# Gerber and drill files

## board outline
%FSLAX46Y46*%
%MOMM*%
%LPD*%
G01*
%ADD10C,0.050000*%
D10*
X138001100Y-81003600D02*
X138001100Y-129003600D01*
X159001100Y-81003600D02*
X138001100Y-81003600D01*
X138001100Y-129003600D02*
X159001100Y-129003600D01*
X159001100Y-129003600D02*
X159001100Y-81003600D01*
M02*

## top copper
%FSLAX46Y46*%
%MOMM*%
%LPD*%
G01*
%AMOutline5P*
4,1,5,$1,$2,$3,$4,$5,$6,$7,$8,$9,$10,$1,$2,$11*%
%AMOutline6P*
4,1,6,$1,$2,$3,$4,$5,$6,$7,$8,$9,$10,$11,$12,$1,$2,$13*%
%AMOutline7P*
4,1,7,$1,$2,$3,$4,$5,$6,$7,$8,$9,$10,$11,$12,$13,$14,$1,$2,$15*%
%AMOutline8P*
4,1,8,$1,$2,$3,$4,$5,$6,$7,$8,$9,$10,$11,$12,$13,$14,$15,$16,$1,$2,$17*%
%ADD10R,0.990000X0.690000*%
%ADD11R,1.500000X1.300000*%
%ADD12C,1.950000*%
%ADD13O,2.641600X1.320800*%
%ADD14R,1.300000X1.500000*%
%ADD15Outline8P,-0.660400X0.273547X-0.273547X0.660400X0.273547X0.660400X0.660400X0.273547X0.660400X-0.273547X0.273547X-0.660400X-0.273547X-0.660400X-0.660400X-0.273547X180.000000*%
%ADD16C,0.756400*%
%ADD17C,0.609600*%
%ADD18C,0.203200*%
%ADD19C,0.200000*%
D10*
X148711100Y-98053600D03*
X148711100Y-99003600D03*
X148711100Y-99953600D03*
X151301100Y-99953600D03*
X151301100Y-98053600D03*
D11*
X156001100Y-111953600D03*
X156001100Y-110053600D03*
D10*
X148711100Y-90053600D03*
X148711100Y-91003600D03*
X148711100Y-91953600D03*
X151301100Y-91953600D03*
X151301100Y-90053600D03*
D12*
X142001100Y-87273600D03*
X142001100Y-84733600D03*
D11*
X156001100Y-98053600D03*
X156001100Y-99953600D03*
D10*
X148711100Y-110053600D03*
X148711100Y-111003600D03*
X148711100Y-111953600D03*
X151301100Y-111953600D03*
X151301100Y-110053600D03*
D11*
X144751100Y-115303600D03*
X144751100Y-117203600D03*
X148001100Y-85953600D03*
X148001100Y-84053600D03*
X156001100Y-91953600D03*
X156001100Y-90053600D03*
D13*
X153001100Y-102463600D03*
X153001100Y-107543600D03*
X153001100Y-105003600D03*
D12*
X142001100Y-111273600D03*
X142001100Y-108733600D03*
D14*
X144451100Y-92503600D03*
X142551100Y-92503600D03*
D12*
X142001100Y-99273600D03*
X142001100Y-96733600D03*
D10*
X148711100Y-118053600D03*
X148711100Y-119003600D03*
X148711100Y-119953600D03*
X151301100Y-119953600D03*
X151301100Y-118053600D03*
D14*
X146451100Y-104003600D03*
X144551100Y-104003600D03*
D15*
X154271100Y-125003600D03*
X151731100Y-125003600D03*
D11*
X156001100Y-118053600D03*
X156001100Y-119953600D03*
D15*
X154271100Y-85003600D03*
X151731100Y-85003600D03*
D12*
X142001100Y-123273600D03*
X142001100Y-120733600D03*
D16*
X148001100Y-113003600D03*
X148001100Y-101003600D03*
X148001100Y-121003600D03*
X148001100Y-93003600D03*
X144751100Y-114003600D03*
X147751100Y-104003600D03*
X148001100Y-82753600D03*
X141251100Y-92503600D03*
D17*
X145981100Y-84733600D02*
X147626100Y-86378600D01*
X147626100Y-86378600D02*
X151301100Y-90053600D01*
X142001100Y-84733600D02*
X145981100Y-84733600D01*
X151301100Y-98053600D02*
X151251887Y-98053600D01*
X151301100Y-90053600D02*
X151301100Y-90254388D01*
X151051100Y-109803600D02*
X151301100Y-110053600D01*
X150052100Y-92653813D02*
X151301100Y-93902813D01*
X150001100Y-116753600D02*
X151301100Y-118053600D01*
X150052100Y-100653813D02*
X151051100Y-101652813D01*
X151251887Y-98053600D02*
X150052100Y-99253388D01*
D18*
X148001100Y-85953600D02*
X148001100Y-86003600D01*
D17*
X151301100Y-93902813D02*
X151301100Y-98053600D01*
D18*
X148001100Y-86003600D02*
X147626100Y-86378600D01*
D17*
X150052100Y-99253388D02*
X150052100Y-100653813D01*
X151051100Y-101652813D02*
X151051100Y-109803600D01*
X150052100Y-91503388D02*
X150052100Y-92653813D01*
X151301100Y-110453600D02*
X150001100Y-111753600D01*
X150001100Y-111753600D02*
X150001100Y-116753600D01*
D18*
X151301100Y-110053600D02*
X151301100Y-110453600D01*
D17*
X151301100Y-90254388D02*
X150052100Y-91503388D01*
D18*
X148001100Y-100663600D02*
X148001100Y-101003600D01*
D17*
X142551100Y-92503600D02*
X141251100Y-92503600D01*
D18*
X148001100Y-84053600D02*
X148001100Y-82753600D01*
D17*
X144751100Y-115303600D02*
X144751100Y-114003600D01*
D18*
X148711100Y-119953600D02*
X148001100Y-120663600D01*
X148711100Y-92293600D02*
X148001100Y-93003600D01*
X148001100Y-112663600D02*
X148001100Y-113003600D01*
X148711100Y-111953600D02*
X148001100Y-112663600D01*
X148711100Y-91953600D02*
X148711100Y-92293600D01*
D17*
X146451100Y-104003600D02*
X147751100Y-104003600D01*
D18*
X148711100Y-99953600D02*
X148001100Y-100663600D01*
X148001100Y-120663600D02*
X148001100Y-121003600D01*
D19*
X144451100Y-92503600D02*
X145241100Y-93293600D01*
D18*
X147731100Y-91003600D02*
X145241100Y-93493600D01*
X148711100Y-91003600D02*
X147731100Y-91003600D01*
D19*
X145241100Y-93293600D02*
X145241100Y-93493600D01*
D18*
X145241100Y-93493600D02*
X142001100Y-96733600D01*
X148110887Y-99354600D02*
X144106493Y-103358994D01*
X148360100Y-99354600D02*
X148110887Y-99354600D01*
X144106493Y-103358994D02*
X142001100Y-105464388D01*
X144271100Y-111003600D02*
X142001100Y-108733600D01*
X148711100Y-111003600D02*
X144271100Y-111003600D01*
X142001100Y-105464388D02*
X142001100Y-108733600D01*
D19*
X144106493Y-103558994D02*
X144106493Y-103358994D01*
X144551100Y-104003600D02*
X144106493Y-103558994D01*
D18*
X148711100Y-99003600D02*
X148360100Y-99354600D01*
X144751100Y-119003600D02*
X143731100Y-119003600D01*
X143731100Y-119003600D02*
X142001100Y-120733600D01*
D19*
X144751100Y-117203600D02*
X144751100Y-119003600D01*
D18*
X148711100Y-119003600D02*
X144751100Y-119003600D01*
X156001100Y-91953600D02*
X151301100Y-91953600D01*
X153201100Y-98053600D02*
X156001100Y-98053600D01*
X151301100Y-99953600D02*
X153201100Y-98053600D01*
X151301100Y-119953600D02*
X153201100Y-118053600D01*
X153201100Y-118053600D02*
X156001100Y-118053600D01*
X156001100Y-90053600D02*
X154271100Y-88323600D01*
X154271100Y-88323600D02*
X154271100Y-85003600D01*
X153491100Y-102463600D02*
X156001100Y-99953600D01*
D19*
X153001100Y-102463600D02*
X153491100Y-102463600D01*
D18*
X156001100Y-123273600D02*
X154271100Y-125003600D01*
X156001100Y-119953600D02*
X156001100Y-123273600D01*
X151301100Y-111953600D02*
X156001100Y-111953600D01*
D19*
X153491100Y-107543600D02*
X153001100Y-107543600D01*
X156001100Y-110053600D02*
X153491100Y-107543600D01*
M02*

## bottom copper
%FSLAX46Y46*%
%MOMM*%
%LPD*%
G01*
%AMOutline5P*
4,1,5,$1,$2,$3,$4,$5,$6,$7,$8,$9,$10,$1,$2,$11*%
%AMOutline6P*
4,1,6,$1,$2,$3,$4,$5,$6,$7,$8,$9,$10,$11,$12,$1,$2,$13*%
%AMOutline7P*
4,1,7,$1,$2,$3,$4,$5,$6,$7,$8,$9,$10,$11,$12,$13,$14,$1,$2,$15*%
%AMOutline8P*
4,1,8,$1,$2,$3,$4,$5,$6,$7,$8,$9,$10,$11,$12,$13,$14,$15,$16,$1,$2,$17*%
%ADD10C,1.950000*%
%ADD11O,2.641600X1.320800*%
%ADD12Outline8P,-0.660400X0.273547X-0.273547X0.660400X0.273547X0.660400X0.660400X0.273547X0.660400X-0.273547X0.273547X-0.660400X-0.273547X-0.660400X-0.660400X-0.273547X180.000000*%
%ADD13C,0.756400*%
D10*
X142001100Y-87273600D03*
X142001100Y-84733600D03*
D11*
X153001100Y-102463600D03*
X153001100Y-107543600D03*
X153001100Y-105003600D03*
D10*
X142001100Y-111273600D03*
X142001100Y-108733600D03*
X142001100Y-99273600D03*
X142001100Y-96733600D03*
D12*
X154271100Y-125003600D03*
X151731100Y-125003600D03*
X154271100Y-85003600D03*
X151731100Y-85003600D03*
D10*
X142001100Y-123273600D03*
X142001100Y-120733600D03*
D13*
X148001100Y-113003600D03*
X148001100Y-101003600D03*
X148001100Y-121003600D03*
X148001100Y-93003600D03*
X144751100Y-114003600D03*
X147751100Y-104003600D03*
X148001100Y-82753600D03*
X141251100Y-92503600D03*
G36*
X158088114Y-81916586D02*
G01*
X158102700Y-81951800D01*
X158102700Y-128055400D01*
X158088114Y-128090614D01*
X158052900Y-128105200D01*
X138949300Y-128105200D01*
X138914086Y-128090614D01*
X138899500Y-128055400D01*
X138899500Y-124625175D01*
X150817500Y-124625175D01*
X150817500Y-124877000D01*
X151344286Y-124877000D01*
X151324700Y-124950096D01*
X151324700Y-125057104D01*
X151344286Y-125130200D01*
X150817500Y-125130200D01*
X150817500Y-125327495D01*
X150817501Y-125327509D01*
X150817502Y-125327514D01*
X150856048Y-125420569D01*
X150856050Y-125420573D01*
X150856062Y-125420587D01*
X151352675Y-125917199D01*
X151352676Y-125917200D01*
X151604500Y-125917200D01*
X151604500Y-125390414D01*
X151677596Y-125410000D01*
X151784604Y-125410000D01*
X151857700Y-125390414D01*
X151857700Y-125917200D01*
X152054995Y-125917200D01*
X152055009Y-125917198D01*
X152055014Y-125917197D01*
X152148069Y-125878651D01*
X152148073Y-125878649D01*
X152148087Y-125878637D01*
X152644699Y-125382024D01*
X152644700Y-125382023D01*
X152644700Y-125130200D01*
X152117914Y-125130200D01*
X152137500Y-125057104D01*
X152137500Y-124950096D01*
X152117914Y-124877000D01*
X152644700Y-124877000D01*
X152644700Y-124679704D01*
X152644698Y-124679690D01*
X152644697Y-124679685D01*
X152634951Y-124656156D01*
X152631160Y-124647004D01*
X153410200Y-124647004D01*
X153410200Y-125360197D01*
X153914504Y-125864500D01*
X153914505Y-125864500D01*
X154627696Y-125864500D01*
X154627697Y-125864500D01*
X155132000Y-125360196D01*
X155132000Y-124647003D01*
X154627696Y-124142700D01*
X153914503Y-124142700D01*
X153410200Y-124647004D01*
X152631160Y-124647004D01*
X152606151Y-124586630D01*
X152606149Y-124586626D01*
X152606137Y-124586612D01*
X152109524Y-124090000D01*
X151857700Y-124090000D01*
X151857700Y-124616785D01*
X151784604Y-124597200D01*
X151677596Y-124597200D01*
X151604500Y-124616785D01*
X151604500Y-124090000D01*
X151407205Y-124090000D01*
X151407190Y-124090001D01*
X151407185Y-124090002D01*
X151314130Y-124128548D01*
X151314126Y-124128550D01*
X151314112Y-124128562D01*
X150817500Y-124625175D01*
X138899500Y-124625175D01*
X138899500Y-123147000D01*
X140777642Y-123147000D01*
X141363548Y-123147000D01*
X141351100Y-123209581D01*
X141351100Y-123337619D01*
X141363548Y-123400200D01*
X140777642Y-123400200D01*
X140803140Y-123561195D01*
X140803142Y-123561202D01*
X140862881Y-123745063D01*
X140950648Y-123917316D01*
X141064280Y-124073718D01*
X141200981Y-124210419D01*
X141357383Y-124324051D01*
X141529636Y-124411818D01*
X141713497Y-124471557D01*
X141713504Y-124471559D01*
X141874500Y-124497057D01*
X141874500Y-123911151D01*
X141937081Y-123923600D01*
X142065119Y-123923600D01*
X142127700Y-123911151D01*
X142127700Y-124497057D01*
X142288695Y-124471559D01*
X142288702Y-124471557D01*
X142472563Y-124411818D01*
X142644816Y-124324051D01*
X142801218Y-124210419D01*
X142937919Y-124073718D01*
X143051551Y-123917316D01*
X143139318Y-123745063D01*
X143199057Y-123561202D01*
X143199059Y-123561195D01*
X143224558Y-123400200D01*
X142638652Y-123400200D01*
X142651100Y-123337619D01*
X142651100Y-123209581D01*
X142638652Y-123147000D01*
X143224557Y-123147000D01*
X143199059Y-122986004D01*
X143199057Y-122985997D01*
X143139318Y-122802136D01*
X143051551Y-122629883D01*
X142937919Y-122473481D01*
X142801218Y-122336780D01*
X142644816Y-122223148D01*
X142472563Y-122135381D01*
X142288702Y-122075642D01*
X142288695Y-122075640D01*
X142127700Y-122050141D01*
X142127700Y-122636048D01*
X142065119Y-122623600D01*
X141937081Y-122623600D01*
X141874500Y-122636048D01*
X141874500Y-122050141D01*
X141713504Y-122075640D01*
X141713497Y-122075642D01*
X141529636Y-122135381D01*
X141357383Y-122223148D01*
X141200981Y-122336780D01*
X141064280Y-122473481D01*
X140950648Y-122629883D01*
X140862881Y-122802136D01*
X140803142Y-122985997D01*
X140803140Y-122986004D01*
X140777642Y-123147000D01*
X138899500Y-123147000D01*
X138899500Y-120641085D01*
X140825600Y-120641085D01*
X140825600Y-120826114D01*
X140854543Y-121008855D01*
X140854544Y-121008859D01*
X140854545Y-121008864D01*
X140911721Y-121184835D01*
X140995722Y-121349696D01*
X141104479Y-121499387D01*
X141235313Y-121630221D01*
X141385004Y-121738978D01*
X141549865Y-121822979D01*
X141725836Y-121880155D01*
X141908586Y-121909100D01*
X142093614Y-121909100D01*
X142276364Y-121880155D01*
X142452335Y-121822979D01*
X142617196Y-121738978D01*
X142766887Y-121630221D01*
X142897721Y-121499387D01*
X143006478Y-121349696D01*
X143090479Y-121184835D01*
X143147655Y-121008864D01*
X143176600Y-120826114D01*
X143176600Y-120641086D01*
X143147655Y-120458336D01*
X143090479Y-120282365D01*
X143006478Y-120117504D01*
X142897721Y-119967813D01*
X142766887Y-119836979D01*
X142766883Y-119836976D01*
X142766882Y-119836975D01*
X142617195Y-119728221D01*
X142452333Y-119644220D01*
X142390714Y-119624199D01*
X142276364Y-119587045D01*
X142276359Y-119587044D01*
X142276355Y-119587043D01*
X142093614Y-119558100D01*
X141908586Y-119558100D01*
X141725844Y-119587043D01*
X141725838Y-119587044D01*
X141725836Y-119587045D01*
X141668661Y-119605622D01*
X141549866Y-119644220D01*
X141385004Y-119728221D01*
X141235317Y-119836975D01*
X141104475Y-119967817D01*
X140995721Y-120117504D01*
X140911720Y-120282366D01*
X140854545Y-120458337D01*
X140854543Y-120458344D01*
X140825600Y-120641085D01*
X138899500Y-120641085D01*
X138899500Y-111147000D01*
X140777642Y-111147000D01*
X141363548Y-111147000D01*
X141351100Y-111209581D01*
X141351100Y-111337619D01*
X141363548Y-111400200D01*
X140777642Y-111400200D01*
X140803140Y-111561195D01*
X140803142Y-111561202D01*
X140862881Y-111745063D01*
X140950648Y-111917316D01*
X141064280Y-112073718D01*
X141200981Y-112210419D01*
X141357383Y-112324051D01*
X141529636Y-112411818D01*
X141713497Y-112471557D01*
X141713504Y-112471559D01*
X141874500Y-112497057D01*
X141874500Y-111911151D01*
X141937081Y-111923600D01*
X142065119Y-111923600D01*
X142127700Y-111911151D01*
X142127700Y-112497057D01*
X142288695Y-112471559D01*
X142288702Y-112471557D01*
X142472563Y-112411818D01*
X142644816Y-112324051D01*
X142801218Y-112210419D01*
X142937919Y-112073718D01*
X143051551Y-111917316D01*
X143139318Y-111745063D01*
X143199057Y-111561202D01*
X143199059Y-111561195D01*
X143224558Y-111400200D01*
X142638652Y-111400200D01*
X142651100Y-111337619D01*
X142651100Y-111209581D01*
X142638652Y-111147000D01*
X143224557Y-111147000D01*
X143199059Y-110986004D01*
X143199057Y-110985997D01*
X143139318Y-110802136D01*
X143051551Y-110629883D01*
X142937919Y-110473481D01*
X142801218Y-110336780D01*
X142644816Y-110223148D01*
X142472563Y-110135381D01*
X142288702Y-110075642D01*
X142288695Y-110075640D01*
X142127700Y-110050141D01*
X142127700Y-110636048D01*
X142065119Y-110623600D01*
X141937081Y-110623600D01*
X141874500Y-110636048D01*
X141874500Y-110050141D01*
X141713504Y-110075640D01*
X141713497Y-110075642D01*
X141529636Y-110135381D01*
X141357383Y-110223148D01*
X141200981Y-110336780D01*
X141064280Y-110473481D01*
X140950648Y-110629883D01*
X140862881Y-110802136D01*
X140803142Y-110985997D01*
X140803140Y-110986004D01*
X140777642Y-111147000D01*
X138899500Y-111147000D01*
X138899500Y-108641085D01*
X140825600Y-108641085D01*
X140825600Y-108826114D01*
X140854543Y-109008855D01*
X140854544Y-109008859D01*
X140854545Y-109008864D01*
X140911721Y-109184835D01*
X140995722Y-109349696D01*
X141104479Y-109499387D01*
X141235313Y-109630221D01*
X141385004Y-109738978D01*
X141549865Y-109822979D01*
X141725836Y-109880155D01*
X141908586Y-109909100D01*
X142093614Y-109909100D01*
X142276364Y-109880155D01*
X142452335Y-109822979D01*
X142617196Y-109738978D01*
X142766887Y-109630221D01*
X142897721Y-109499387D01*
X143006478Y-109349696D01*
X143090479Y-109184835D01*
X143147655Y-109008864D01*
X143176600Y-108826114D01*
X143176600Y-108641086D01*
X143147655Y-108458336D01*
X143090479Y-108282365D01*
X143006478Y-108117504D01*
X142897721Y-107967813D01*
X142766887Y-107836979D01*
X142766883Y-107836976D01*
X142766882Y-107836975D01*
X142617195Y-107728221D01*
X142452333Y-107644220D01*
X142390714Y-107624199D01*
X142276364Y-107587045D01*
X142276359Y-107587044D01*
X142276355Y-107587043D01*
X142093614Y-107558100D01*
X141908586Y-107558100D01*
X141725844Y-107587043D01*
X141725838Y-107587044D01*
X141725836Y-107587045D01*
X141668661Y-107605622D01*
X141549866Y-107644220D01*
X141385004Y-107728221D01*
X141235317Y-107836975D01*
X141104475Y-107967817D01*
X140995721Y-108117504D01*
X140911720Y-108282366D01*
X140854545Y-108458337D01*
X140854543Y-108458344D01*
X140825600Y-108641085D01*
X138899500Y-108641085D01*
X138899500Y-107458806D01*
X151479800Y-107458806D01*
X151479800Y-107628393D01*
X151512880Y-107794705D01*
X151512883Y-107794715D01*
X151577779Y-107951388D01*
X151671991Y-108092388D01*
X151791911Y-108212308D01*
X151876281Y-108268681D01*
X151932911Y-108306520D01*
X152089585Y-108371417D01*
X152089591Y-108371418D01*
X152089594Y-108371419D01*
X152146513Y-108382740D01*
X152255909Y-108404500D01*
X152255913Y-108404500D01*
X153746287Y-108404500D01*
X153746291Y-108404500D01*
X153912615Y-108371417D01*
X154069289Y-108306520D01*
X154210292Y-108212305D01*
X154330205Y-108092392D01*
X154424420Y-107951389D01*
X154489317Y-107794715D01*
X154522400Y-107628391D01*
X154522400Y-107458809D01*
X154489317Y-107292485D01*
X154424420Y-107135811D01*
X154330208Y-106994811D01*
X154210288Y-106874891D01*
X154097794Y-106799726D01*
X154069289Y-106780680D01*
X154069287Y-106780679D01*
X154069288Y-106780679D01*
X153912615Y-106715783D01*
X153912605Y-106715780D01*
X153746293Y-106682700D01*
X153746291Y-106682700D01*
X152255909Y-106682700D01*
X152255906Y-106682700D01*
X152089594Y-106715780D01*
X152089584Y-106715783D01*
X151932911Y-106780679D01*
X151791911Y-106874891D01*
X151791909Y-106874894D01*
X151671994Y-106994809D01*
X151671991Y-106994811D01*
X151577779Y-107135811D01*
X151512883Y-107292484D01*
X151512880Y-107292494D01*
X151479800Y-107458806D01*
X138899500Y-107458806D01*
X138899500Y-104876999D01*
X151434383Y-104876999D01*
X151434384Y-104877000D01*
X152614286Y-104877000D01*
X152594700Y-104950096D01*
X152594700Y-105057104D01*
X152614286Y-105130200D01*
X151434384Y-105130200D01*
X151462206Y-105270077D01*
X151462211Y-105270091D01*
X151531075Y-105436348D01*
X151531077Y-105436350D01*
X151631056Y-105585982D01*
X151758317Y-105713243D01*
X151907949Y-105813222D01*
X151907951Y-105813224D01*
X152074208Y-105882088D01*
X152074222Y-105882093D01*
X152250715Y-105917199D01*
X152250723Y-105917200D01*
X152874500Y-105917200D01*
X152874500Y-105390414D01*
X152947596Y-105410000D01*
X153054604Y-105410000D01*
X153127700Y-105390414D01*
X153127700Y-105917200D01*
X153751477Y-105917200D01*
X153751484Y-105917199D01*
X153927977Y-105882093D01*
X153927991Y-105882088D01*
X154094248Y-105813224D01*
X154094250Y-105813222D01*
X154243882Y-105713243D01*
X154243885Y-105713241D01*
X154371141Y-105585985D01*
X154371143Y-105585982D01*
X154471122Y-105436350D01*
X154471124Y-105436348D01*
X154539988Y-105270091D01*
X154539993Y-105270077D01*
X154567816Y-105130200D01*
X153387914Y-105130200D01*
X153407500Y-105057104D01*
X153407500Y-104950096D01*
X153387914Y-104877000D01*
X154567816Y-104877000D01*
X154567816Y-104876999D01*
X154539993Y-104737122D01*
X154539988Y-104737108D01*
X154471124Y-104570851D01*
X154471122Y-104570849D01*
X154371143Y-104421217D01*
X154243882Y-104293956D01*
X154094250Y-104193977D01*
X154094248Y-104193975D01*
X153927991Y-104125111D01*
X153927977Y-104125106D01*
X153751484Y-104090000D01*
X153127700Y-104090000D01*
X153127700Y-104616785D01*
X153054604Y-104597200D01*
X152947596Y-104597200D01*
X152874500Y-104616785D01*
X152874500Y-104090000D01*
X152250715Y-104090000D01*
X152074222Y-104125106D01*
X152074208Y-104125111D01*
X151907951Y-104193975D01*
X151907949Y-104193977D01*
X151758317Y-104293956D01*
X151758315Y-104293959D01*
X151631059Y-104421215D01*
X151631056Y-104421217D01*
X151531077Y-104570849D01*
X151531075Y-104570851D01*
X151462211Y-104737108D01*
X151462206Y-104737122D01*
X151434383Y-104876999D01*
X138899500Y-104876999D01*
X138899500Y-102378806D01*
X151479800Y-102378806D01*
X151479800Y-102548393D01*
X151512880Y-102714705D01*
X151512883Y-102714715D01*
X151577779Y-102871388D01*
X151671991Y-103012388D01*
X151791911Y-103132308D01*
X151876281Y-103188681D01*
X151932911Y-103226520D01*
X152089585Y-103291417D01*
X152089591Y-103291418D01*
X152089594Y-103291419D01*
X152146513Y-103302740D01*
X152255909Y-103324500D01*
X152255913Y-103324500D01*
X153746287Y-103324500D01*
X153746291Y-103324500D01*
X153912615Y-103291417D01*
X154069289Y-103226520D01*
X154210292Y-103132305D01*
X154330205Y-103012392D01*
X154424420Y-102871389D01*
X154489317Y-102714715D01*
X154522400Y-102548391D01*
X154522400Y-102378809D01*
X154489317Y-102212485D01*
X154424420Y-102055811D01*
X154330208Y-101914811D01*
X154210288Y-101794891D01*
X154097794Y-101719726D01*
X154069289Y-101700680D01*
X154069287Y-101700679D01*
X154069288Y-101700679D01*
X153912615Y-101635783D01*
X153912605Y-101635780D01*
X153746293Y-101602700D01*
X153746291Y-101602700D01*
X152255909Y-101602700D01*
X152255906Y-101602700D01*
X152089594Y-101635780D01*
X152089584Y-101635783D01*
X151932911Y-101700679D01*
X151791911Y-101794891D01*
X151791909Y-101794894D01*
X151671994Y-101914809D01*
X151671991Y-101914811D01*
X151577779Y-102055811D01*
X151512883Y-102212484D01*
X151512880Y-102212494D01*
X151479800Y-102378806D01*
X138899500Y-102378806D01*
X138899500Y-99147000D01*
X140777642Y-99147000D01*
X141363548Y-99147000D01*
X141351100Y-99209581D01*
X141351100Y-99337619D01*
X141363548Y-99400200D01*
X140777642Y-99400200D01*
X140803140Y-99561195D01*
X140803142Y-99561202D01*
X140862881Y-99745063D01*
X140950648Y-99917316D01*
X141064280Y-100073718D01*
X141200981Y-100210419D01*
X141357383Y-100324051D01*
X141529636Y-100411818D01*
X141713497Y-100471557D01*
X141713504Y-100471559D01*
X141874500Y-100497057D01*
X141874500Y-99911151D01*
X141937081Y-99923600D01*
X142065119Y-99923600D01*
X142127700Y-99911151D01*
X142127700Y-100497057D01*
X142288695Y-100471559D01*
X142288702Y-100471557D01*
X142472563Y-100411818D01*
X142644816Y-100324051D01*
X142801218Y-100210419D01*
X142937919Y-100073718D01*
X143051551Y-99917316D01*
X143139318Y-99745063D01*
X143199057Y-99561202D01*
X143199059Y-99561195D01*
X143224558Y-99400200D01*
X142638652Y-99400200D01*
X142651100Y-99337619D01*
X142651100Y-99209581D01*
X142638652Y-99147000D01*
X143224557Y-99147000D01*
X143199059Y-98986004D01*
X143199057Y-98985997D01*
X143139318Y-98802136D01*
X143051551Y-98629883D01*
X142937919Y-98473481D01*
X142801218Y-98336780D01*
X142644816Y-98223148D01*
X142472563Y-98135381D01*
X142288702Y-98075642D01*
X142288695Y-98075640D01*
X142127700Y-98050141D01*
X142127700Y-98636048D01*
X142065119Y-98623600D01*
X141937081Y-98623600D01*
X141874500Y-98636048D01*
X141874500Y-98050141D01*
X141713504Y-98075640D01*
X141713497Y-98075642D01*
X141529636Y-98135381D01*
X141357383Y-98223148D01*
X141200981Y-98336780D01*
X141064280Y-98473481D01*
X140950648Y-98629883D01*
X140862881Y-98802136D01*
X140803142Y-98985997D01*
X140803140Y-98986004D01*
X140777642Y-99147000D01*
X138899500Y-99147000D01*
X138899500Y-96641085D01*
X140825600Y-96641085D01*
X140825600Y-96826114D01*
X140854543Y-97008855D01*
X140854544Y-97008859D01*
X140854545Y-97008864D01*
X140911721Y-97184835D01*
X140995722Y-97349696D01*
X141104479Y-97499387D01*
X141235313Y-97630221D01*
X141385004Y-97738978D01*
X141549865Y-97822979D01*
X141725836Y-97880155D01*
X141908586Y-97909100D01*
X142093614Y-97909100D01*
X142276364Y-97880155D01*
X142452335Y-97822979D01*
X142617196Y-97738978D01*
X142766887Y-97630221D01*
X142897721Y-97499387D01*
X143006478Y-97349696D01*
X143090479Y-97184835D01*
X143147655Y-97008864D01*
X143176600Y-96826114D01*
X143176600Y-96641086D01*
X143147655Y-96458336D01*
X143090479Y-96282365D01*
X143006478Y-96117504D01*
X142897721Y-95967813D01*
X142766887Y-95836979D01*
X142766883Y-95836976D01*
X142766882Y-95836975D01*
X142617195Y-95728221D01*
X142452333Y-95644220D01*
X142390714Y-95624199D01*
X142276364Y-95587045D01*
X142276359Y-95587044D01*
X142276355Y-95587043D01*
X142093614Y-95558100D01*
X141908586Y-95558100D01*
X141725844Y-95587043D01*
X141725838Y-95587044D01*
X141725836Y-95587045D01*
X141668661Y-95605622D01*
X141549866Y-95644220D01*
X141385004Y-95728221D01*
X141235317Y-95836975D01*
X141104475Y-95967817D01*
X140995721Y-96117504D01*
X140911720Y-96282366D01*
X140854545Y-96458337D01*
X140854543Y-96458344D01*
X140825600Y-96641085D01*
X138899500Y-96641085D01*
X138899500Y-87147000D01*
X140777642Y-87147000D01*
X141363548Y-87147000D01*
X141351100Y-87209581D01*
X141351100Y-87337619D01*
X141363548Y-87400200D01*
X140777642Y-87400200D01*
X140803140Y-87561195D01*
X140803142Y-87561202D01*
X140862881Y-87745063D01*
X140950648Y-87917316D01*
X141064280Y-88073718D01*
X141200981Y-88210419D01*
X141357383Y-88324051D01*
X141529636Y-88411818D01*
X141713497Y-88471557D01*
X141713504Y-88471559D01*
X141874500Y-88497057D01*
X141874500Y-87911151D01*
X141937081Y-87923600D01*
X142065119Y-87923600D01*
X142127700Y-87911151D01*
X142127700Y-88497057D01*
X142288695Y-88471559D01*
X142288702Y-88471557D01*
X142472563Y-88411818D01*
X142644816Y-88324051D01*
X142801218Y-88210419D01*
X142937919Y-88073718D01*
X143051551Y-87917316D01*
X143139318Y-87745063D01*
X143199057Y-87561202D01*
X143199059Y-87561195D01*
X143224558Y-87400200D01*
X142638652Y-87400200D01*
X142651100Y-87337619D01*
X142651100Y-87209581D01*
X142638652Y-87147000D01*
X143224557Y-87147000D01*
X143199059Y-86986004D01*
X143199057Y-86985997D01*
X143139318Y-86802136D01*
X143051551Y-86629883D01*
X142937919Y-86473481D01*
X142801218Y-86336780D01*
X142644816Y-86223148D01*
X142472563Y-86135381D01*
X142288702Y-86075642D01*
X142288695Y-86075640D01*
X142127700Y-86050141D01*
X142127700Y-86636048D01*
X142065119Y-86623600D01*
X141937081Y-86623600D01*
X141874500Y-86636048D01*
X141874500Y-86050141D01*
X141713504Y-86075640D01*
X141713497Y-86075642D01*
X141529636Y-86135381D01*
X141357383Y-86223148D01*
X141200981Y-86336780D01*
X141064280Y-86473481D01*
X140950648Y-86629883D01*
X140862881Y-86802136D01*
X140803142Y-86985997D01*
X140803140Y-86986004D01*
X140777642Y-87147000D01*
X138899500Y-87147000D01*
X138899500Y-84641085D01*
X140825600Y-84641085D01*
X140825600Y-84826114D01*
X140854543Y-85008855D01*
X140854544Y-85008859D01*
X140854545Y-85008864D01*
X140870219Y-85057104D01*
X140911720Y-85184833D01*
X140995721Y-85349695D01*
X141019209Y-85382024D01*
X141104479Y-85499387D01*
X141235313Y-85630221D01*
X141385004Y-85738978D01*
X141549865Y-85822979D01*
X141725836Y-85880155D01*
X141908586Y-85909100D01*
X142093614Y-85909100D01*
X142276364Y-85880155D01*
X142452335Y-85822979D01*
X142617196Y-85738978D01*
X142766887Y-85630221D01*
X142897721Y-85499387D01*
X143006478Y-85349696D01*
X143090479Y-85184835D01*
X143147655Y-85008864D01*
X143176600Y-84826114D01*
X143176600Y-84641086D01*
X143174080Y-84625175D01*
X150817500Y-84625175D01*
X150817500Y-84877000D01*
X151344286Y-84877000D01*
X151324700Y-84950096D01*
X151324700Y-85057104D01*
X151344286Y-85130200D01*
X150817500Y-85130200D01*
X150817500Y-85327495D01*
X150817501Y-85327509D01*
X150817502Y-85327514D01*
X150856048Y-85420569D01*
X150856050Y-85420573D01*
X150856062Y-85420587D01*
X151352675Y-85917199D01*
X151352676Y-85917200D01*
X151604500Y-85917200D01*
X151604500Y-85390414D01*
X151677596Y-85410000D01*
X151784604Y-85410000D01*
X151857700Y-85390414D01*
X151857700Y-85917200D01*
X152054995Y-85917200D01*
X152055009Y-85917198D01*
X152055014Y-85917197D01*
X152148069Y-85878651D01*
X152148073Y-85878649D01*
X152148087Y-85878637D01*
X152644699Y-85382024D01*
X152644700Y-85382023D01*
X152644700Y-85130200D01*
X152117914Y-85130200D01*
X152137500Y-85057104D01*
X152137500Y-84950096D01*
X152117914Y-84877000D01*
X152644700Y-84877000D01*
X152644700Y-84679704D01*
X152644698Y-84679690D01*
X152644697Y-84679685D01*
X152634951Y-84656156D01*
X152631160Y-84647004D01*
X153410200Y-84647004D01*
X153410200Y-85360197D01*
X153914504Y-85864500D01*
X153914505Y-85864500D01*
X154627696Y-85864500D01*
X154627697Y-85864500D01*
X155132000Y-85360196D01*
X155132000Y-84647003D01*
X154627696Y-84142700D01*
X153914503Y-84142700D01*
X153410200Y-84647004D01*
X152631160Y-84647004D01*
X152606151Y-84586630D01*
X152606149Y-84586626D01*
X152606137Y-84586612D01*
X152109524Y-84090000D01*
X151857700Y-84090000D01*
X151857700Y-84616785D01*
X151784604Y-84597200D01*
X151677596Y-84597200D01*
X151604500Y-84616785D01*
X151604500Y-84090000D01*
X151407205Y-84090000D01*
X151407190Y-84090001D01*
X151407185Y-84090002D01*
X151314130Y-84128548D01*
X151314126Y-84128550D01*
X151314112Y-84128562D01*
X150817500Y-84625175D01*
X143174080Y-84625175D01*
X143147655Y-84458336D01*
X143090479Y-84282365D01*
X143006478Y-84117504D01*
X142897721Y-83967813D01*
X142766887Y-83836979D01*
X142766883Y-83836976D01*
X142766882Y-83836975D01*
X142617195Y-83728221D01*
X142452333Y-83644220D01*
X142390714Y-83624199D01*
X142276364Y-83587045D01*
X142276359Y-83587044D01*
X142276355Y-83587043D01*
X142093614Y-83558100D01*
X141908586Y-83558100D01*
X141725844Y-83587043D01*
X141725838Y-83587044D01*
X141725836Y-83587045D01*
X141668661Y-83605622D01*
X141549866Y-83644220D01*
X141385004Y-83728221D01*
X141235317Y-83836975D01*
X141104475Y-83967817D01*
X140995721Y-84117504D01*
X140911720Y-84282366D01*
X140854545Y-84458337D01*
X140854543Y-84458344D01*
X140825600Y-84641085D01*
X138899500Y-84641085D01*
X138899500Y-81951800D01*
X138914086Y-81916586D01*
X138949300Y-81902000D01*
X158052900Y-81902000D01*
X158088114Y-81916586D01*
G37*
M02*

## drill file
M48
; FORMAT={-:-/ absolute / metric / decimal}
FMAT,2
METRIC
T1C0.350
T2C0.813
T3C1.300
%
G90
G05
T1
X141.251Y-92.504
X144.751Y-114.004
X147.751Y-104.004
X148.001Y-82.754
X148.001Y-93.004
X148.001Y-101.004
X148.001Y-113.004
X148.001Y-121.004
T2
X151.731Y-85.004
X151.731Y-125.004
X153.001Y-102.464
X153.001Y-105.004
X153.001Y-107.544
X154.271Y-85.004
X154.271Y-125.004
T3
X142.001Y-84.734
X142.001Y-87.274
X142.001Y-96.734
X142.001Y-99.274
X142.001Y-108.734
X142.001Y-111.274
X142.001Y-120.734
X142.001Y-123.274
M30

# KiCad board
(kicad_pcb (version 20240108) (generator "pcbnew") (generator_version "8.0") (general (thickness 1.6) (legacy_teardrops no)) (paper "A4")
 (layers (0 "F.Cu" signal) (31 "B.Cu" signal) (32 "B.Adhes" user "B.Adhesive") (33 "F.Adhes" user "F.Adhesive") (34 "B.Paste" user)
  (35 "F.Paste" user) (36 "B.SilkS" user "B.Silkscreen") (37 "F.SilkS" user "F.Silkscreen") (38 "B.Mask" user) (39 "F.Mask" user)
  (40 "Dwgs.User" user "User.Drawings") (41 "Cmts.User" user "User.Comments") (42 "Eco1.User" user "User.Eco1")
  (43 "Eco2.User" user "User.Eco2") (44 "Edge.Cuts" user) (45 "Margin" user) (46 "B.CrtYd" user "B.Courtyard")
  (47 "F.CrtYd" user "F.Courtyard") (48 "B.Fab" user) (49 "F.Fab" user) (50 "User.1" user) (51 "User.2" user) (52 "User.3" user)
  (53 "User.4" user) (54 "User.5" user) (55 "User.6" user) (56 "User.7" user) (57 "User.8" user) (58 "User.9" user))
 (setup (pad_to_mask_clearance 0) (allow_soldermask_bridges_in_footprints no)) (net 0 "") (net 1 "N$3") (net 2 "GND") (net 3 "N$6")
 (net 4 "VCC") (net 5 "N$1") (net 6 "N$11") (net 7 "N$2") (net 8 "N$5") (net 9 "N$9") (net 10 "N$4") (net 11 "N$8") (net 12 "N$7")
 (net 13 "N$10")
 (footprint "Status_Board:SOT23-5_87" (layer "F.Cu") (at 150.0011 99.0036 -90)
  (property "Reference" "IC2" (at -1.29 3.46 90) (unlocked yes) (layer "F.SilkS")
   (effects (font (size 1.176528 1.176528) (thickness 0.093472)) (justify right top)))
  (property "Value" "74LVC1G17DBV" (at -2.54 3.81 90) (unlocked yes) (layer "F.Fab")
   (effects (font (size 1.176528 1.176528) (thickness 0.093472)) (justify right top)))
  (pad "1" smd rect (at -0.95 1.29 270) (size 0.69 0.99) (layers "F.Cu" "F.Paste" "F.Mask") (solder_mask_margin 0.1016)
   (thermal_bridge_angle 0))
  (pad "2" smd rect (at 0 1.29 270) (size 0.69 0.99) (layers "F.Cu" "F.Paste" "F.Mask") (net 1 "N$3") (solder_mask_margin 0.1016)
   (thermal_bridge_angle 0))
  (pad "3" smd rect (at 0.95 1.29 270) (size 0.69 0.99) (layers "F.Cu" "F.Paste" "F.Mask") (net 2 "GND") (solder_mask_margin 0.1016)
   (thermal_bridge_angle 0))
  (pad "4" smd rect (at 0.95 -1.3 270) (size 0.69 0.99) (layers "F.Cu" "F.Paste" "F.Mask") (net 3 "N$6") (solder_mask_margin 0.1016)
   (thermal_bridge_angle 0))
  (pad "5" smd rect (at -0.95 -1.3 270) (size 0.69 0.99) (layers "F.Cu" "F.Paste" "F.Mask") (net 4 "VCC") (solder_mask_margin 0.1016)
   (thermal_bridge_angle 0)))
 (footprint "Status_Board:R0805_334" (layer "F.Cu") (at 156.0011 111.0036 90)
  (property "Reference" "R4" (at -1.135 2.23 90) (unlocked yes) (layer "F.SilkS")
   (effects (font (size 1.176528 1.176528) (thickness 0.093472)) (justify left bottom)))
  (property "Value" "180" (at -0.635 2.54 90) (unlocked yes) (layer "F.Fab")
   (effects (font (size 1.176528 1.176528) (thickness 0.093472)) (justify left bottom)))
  (pad "1" smd rect (at -0.95 0 90) (size 1.3 1.5) (layers "F.Cu" "F.Paste" "F.Mask") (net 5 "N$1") (solder_mask_margin 0.1016)
   (thermal_bridge_angle 0))
  (pad "2" smd rect (at 0.95 0 90) (size 1.3 1.5) (layers "F.Cu" "F.Paste" "F.Mask") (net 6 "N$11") (solder_mask_margin 0.1016)
   (thermal_bridge_angle 0)))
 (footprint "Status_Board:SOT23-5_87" (layer "F.Cu") (at 150.0011 91.0036 -90)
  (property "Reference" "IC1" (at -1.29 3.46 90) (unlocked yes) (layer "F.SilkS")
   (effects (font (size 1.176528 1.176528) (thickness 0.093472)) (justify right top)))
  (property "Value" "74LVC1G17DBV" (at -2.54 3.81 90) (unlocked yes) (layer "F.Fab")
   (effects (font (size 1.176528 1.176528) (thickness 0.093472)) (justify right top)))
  (pad "1" smd rect (at -0.95 1.29 270) (size 0.69 0.99) (layers "F.Cu" "F.Paste" "F.Mask") (solder_mask_margin 0.1016)
   (thermal_bridge_angle 0))
  (pad "2" smd rect (at 0 1.29 270) (size 0.69 0.99) (layers "F.Cu" "F.Paste" "F.Mask") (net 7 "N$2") (solder_mask_margin 0.1016)
   (thermal_bridge_angle 0))
  (pad "3" smd rect (at 0.95 1.29 270) (size 0.69 0.99) (layers "F.Cu" "F.Paste" "F.Mask") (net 2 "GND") (solder_mask_margin 0.1016)
   (thermal_bridge_angle 0))
  (pad "4" smd rect (at 0.95 -1.3 270) (size 0.69 0.99) (layers "F.Cu" "F.Paste" "F.Mask") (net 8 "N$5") (solder_mask_margin 0.1016)
   (thermal_bridge_angle 0))
  (pad "5" smd rect (at -0.95 -1.3 270) (size 0.69 0.99) (layers "F.Cu" "F.Paste" "F.Mask") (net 4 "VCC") (solder_mask_margin 0.1016)
   (thermal_bridge_angle 0)))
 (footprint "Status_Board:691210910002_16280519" (layer "F.Cu") (at 142.0011 86.0036 90)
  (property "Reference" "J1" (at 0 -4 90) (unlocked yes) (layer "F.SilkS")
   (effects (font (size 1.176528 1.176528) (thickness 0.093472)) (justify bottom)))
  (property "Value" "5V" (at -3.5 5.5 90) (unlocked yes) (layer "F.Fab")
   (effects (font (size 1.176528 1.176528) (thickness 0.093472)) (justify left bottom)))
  (pad "1" thru_hole circle (at -1.27 0 90) (size 1.95 1.95) (drill 1.3) (layers "*.Cu" "*.Mask") (remove_unused_layers no) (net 2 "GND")
   (solder_mask_margin 0.1016) (thermal_bridge_angle 0))
  (pad "2" thru_hole circle (at 1.27 0 90) (size 1.95 1.95) (drill 1.3) (layers "*.Cu" "*.Mask") (remove_unused_layers no) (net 4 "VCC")
   (solder_mask_margin 0.1016) (thermal_bridge_angle 0)))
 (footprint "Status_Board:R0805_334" (layer "F.Cu") (at 156.0011 99.0036 -90)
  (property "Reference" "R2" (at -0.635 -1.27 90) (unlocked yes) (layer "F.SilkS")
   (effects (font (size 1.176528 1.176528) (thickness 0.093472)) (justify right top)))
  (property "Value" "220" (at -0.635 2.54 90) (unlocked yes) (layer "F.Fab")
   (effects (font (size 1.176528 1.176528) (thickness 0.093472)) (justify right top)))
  (pad "1" smd rect (at -0.95 0 270) (size 1.3 1.5) (layers "F.Cu" "F.Paste" "F.Mask") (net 3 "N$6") (solder_mask_margin 0.1016)
   (thermal_bridge_angle 0))
  (pad "2" smd rect (at 0.95 0 270) (size 1.3 1.5) (layers "F.Cu" "F.Paste" "F.Mask") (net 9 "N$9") (solder_mask_margin 0.1016)
   (thermal_bridge_angle 0)))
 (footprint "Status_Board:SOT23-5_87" (layer "F.Cu") (at 150.0011 111.0036 -90)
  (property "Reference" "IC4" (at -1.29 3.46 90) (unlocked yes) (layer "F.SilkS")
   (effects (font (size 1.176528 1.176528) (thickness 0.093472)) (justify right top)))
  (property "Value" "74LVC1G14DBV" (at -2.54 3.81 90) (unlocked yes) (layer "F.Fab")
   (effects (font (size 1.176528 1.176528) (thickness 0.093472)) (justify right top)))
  (pad "1" smd rect (at -0.95 1.29 270) (size 0.69 0.99) (layers "F.Cu" "F.Paste" "F.Mask") (solder_mask_margin 0.1016)
   (thermal_bridge_angle 0))
  (pad "2" smd rect (at 0 1.29 270) (size 0.69 0.99) (layers "F.Cu" "F.Paste" "F.Mask") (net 1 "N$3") (solder_mask_margin 0.1016)
   (thermal_bridge_angle 0))
  (pad "3" smd rect (at 0.95 1.29 270) (size 0.69 0.99) (layers "F.Cu" "F.Paste" "F.Mask") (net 2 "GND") (solder_mask_margin 0.1016)
   (thermal_bridge_angle 0))
  (pad "4" smd rect (at 0.95 -1.3 270) (size 0.69 0.99) (layers "F.Cu" "F.Paste" "F.Mask") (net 5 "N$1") (solder_mask_margin 0.1016)
   (thermal_bridge_angle 0))
  (pad "5" smd rect (at -0.95 -1.3 270) (size 0.69 0.99) (layers "F.Cu" "F.Paste" "F.Mask") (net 4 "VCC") (solder_mask_margin 0.1016)
   (thermal_bridge_angle 0)))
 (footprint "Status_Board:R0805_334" (layer "F.Cu") (at 144.7511 116.2536 -90)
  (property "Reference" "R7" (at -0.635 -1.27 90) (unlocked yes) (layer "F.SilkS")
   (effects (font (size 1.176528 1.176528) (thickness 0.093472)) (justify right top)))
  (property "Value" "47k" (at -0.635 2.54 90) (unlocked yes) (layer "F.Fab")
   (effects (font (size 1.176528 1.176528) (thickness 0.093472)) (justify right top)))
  (pad "1" smd rect (at -0.95 0 270) (size 1.3 1.5) (layers "F.Cu" "F.Paste" "F.Mask") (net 2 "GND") (solder_mask_margin 0.1016)
   (thermal_bridge_angle 0))
  (pad "2" smd rect (at 0.95 0 270) (size 1.3 1.5) (layers "F.Cu" "F.Paste" "F.Mask") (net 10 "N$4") (solder_mask_margin 0.1016)
   (thermal_bridge_angle 0)))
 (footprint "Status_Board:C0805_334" (layer "F.Cu") (at 148.0011 85.0036 90)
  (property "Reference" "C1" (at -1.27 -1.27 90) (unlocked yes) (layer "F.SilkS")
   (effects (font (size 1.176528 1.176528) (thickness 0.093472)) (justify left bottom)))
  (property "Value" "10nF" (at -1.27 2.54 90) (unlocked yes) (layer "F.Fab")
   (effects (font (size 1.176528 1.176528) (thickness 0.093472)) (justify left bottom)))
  (pad "1" smd rect (at -0.95 0 90) (size 1.3 1.5) (layers "F.Cu" "F.Paste" "F.Mask") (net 4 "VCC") (solder_mask_margin 0.1016)
   (thermal_bridge_angle 0))
  (pad "2" smd rect (at 0.95 0 90) (size 1.3 1.5) (layers "F.Cu" "F.Paste" "F.Mask") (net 2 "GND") (solder_mask_margin 0.1016)
   (thermal_bridge_angle 0)))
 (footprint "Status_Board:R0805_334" (layer "F.Cu") (at 156.0011 91.0036 90)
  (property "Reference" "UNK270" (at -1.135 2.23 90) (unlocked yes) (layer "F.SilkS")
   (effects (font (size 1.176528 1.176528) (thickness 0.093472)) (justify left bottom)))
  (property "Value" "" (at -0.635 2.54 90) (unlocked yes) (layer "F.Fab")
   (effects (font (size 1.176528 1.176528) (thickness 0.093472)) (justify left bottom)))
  (pad "1" smd rect (at -0.95 0 90) (size 1.3 1.5) (layers "F.Cu" "F.Paste" "F.Mask") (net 8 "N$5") (solder_mask_margin 0.1016)
   (thermal_bridge_angle 0))
  (pad "2" smd rect (at 0.95 0 90) (size 1.3 1.5) (layers "F.Cu" "F.Paste" "F.Mask") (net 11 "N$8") (solder_mask_margin 0.1016)
   (thermal_bridge_angle 0)))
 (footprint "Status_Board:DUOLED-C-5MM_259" (layer "F.Cu") (at 153.0011 105.0036 90)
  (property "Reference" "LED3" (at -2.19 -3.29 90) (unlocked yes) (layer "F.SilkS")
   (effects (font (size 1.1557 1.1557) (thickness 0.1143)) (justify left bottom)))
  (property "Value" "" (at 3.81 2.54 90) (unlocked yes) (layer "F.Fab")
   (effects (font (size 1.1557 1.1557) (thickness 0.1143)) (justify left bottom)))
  (pad "AR" thru_hole oval (at 2.54 0 180) (size 2.6416 1.3208) (drill 0.8128) (layers "*.Cu" "*.Mask") (remove_unused_layers no)
   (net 9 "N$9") (solder_mask_margin 0.1016) (thermal_bridge_angle 0))
  (pad "AX" thru_hole oval (at -2.54 0 180) (size 2.6416 1.3208) (drill 0.8128) (layers "*.Cu" "*.Mask") (remove_unused_layers no)
   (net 6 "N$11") (solder_mask_margin 0.1016) (thermal_bridge_angle 0))
  (pad "C" thru_hole oval (at 0 0 180) (size 2.6416 1.3208) (drill 0.8128) (layers "*.Cu" "*.Mask") (remove_unused_layers no) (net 2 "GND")
   (solder_mask_margin 0.1016) (thermal_bridge_angle 0)))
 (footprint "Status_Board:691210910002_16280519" (layer "F.Cu") (at 142.0011 110.0036 90)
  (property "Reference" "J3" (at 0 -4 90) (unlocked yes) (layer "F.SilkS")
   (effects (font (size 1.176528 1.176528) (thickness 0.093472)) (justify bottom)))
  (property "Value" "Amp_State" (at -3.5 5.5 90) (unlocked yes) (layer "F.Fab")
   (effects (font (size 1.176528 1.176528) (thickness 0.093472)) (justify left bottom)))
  (pad "1" thru_hole circle (at -1.27 0 90) (size 1.95 1.95) (drill 1.3) (layers "*.Cu" "*.Mask") (remove_unused_layers no) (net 2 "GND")
   (solder_mask_margin 0.1016) (thermal_bridge_angle 0))
  (pad "2" thru_hole circle (at 1.27 0 90) (size 1.95 1.95) (drill 1.3) (layers "*.Cu" "*.Mask") (remove_unused_layers no) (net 1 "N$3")
   (solder_mask_margin 0.1016) (thermal_bridge_angle 0)))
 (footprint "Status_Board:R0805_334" (layer "F.Cu") (at 143.5011 92.5036 180)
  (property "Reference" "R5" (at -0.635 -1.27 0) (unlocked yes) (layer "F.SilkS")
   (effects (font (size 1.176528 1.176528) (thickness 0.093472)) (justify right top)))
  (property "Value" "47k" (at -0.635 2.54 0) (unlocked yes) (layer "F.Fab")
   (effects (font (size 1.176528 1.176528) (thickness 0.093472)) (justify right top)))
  (pad "1" smd rect (at -0.95 0 180) (size 1.3 1.5) (layers "F.Cu" "F.Paste" "F.Mask") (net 7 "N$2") (solder_mask_margin 0.1016)
   (thermal_bridge_angle 0))
  (pad "2" smd rect (at 0.95 0 180) (size 1.3 1.5) (layers "F.Cu" "F.Paste" "F.Mask") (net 2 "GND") (solder_mask_margin 0.1016)
   (thermal_bridge_angle 0)))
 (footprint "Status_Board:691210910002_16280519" (layer "F.Cu") (at 142.0011 98.0036 90)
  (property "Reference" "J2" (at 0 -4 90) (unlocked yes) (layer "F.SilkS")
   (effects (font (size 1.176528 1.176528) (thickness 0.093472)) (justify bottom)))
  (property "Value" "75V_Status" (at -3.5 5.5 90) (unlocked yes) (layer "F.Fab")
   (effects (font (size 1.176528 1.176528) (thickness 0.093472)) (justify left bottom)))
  (pad "1" thru_hole circle (at -1.27 0 90) (size 1.95 1.95) (drill 1.3) (layers "*.Cu" "*.Mask") (remove_unused_layers no) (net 2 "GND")
   (solder_mask_margin 0.1016) (thermal_bridge_angle 0))
  (pad "2" thru_hole circle (at 1.27 0 90) (size 1.95 1.95) (drill 1.3) (layers "*.Cu" "*.Mask") (remove_unused_layers no) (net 7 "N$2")
   (solder_mask_margin 0.1016) (thermal_bridge_angle 0)))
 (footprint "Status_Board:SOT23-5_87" (layer "F.Cu") (at 150.0011 119.0036 -90)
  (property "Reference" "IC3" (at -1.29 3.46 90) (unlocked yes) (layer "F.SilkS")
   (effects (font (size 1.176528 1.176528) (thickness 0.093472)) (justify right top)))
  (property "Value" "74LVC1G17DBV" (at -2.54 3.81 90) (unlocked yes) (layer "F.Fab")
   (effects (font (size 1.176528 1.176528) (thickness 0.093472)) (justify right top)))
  (pad "1" smd rect (at -0.95 1.29 270) (size 0.69 0.99) (layers "F.Cu" "F.Paste" "F.Mask") (solder_mask_margin 0.1016)
   (thermal_bridge_angle 0))
  (pad "2" smd rect (at 0 1.29 270) (size 0.69 0.99) (layers "F.Cu" "F.Paste" "F.Mask") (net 10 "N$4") (solder_mask_margin 0.1016)
   (thermal_bridge_angle 0))
  (pad "3" smd rect (at 0.95 1.29 270) (size 0.69 0.99) (layers "F.Cu" "F.Paste" "F.Mask") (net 2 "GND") (solder_mask_margin 0.1016)
   (thermal_bridge_angle 0))
  (pad "4" smd rect (at 0.95 -1.3 270) (size 0.69 0.99) (layers "F.Cu" "F.Paste" "F.Mask") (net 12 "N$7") (solder_mask_margin 0.1016)
   (thermal_bridge_angle 0))
  (pad "5" smd rect (at -0.95 -1.3 270) (size 0.69 0.99) (layers "F.Cu" "F.Paste" "F.Mask") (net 4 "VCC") (solder_mask_margin 0.1016)
   (thermal_bridge_angle 0)))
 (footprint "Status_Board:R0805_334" (layer "F.Cu") (at 145.5011 104.0036 180)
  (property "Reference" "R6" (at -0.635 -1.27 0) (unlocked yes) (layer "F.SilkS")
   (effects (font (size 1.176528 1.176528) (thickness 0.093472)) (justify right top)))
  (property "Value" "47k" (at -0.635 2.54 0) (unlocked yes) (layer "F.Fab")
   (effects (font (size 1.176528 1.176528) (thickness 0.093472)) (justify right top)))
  (pad "1" smd rect (at -0.95 0 180) (size 1.3 1.5) (layers "F.Cu" "F.Paste" "F.Mask") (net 2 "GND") (solder_mask_margin 0.1016)
   (thermal_bridge_angle 0))
  (pad "2" smd rect (at 0.95 0 180) (size 1.3 1.5) (layers "F.Cu" "F.Paste" "F.Mask") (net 1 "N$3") (solder_mask_margin 0.1016)
   (thermal_bridge_angle 0)))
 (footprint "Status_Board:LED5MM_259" (layer "F.Cu") (at 153.0011 125.0036 180)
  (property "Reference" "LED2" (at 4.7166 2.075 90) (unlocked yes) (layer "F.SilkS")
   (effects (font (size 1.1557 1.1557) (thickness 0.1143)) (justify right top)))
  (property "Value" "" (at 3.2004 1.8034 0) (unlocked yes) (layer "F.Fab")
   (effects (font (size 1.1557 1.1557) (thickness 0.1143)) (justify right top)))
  (pad "A" thru_hole roundrect (at -1.27 0 180) (size 1.3208 1.3208) (drill 0.8128) (layers "*.Cu" "*.Mask") (remove_unused_layers no)
   (roundrect_rratio 0.25) (chamfer_ratio 0.2928932188) (chamfer top_left top_right bottom_left bottom_right) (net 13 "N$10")
   (solder_mask_margin 0.1016) (thermal_bridge_angle 0))
  (pad "K" thru_hole roundrect (at 1.27 0 180) (size 1.3208 1.3208) (drill 0.8128) (layers "*.Cu" "*.Mask") (remove_unused_layers no)
   (roundrect_rratio 0.25) (chamfer_ratio 0.2928932188) (chamfer top_left top_right bottom_left bottom_right) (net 2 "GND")
   (solder_mask_margin 0.1016) (thermal_bridge_angle 0)))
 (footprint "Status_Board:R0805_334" (layer "F.Cu") (at 156.0011 119.0036 -90)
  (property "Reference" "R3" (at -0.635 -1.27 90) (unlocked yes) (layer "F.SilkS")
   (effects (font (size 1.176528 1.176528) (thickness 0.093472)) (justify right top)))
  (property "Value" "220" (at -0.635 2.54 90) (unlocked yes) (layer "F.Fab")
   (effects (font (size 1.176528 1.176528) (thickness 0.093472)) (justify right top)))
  (pad "1" smd rect (at -0.95 0 270) (size 1.3 1.5) (layers "F.Cu" "F.Paste" "F.Mask") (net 12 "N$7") (solder_mask_margin 0.1016)
   (thermal_bridge_angle 0))
  (pad "2" smd rect (at 0.95 0 270) (size 1.3 1.5) (layers "F.Cu" "F.Paste" "F.Mask") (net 13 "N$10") (solder_mask_margin 0.1016)
   (thermal_bridge_angle 0)))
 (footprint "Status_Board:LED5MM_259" (layer "F.Cu") (at 153.0011 85.0036 180)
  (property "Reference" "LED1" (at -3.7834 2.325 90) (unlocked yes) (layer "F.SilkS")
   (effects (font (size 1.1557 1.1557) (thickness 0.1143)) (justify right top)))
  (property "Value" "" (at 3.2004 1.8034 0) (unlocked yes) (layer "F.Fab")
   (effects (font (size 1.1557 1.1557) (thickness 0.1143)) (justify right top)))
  (pad "A" thru_hole roundrect (at -1.27 0 180) (size 1.3208 1.3208) (drill 0.8128) (layers "*.Cu" "*.Mask") (remove_unused_layers no)
   (roundrect_rratio 0.25) (chamfer_ratio 0.2928932188) (chamfer top_left top_right bottom_left bottom_right) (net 11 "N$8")
   (solder_mask_margin 0.1016) (thermal_bridge_angle 0))
  (pad "K" thru_hole roundrect (at 1.27 0 180) (size 1.3208 1.3208) (drill 0.8128) (layers "*.Cu" "*.Mask") (remove_unused_layers no)
   (roundrect_rratio 0.25) (chamfer_ratio 0.2928932188) (chamfer top_left top_right bottom_left bottom_right) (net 2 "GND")
   (solder_mask_margin 0.1016) (thermal_bridge_angle 0)))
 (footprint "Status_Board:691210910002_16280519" (layer "F.Cu") (at 142.0011 122.0036 90)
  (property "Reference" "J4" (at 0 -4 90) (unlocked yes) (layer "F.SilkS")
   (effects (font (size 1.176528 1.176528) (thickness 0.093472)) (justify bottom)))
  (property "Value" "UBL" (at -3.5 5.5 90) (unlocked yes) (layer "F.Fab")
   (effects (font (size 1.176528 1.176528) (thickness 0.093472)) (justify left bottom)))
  (pad "1" thru_hole circle (at -1.27 0 90) (size 1.95 1.95) (drill 1.3) (layers "*.Cu" "*.Mask") (remove_unused_layers no) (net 2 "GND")
   (solder_mask_margin 0.1016) (thermal_bridge_angle 0))
  (pad "2" thru_hole circle (at 1.27 0 90) (size 1.95 1.95) (drill 1.3) (layers "*.Cu" "*.Mask") (remove_unused_layers no) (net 10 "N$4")
   (solder_mask_margin 0.1016) (thermal_bridge_angle 0)))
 (gr_line (start 138.0011 81.0036) (end 138.0011 129.0036) (stroke (width 0.05) (type solid)) (layer "Edge.Cuts"))
 (gr_line (start 159.0011 81.0036) (end 138.0011 81.0036) (stroke (width 0.05) (type solid)) (layer "Edge.Cuts"))
 (gr_line (start 138.0011 129.0036) (end 159.0011 129.0036) (stroke (width 0.05) (type solid)) (layer "Edge.Cuts"))
 (gr_line (start 159.0011 129.0036) (end 159.0011 81.0036) (stroke (width 0.05) (type solid)) (layer "Edge.Cuts"))
 (segment (start 145.9811 84.7336) (end 147.6261 86.3786) (width 0.6096) (layer "F.Cu") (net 4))
 (segment (start 147.6261 86.3786) (end 151.3011 90.0536) (width 0.6096) (layer "F.Cu") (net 4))
 (segment (start 142.0011 84.7336) (end 145.9811 84.7336) (width 0.6096) (layer "F.Cu") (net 4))
 (segment (start 151.3011 98.0536) (end 151.251887 98.0536) (width 0.6096) (layer "F.Cu") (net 4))
 (segment (start 151.3011 90.0536) (end 151.3011 90.254388) (width 0.6096) (layer "F.Cu") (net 4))
 (segment (start 151.0511 109.8036) (end 151.3011 110.0536) (width 0.6096) (layer "F.Cu") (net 4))
 (segment (start 150.0521 92.653813) (end 151.3011 93.902813) (width 0.6096) (layer "F.Cu") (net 4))
 (segment (start 150.0011 116.7536) (end 151.3011 118.0536) (width 0.6096) (layer "F.Cu") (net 4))
 (segment (start 150.0521 100.653813) (end 151.0511 101.652813) (width 0.6096) (layer "F.Cu") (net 4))
 (segment (start 151.251887 98.0536) (end 150.0521 99.253388) (width 0.6096) (layer "F.Cu") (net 4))
 (segment (start 148.0011 85.9536) (end 148.0011 86.0036) (width 0.2032) (layer "F.Cu") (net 4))
 (segment (start 151.3011 93.902813) (end 151.3011 98.0536) (width 0.6096) (layer "F.Cu") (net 4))
 (segment (start 148.0011 86.0036) (end 147.6261 86.3786) (width 0.2032) (layer "F.Cu") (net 4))
 (segment (start 150.0521 99.253388) (end 150.0521 100.653813) (width 0.6096) (layer "F.Cu") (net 4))
 (segment (start 151.0511 101.652813) (end 151.0511 109.8036) (width 0.6096) (layer "F.Cu") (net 4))
 (segment (start 150.0521 91.503388) (end 150.0521 92.653813) (width 0.6096) (layer "F.Cu") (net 4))
 (segment (start 151.3011 110.4536) (end 150.0011 111.7536) (width 0.6096) (layer "F.Cu") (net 4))
 (segment (start 150.0011 111.7536) (end 150.0011 116.7536) (width 0.6096) (layer "F.Cu") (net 4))
 (segment (start 151.3011 110.0536) (end 151.3011 110.4536) (width 0.2032) (layer "F.Cu") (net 4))
 (segment (start 151.3011 90.254388) (end 150.0521 91.503388) (width 0.6096) (layer "F.Cu") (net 4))
 (segment (start 148.0011 100.6636) (end 148.0011 101.0036) (width 0.2032) (layer "F.Cu") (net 2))
 (segment (start 142.5511 92.5036) (end 141.2511 92.5036) (width 0.6096) (layer "F.Cu") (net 2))
 (segment (start 148.0011 84.0536) (end 148.0011 82.7536) (width 0.2032) (layer "F.Cu") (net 2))
 (segment (start 144.7511 115.3036) (end 144.7511 114.0036) (width 0.6096) (layer "F.Cu") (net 2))
 (segment (start 148.7111 119.9536) (end 148.0011 120.6636) (width 0.2032) (layer "F.Cu") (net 2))
 (segment (start 148.7111 92.2936) (end 148.0011 93.0036) (width 0.2032) (layer "F.Cu") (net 2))
 (segment (start 148.0011 112.6636) (end 148.0011 113.0036) (width 0.2032) (layer "F.Cu") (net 2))
 (segment (start 148.7111 111.9536) (end 148.0011 112.6636) (width 0.2032) (layer "F.Cu") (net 2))
 (segment (start 148.7111 91.9536) (end 148.7111 92.2936) (width 0.2032) (layer "F.Cu") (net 2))
 (segment (start 146.4511 104.0036) (end 147.7511 104.0036) (width 0.6096) (layer "F.Cu") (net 2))
 (segment (start 148.7111 99.9536) (end 148.0011 100.6636) (width 0.2032) (layer "F.Cu") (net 2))
 (segment (start 148.0011 120.6636) (end 148.0011 121.0036) (width 0.2032) (layer "F.Cu") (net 2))
 (via (at 148.0011 113.0036) (size 0.7564) (drill 0.35) (layers "F.Cu" "B.Cu") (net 2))
 (via (at 148.0011 101.0036) (size 0.7564) (drill 0.35) (layers "F.Cu" "B.Cu") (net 2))
 (via (at 148.0011 121.0036) (size 0.7564) (drill 0.35) (layers "F.Cu" "B.Cu") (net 2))
 (via (at 148.0011 93.0036) (size 0.7564) (drill 0.35) (layers "F.Cu" "B.Cu") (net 2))
 (via (at 144.7511 114.0036) (size 0.7564) (drill 0.35) (layers "F.Cu" "B.Cu") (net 2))
 (via (at 147.7511 104.0036) (size 0.7564) (drill 0.35) (layers "F.Cu" "B.Cu") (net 2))
 (via (at 148.0011 82.7536) (size 0.7564) (drill 0.35) (layers "F.Cu" "B.Cu") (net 2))
 (via (at 141.2511 92.5036) (size 0.7564) (drill 0.35) (layers "F.Cu" "B.Cu") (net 2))
 (segment (start 144.4511 92.5036) (end 145.2411 93.2936) (width 0.2) (layer "F.Cu") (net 7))
 (segment (start 147.7311 91.0036) (end 145.2411 93.4936) (width 0.2032) (layer "F.Cu") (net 7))
 (segment (start 148.7111 91.0036) (end 147.7311 91.0036) (width 0.2032) (layer "F.Cu") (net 7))
 (segment (start 145.2411 93.2936) (end 145.2411 93.4936) (width 0.2) (layer "F.Cu") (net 7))
 (segment (start 145.2411 93.4936) (end 142.0011 96.7336) (width 0.2032) (layer "F.Cu") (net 7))
 (segment (start 148.110887 99.3546) (end 144.106493 103.358994) (width 0.2032) (layer "F.Cu") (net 1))
 (segment (start 148.3601 99.3546) (end 148.110887 99.3546) (width 0.2032) (layer "F.Cu") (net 1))
 (segment (start 144.106493 103.358994) (end 142.0011 105.464388) (width 0.2032) (layer "F.Cu") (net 1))
 (segment (start 144.2711 111.0036) (end 142.0011 108.7336) (width 0.2032) (layer "F.Cu") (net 1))
 (segment (start 148.7111 111.0036) (end 144.2711 111.0036) (width 0.2032) (layer "F.Cu") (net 1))
 (segment (start 142.0011 105.464388) (end 142.0011 108.7336) (width 0.2032) (layer "F.Cu") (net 1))
 (segment (start 144.106493 103.558994) (end 144.106493 103.358994) (width 0.2) (layer "F.Cu") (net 1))
 (segment (start 144.5511 104.0036) (end 144.106493 103.558994) (width 0.2) (layer "F.Cu") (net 1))
 (segment (start 148.7111 99.0036) (end 148.3601 99.3546) (width 0.2032) (layer "F.Cu") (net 1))
 (segment (start 144.7511 119.0036) (end 143.7311 119.0036) (width 0.2032) (layer "F.Cu") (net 10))
 (segment (start 143.7311 119.0036) (end 142.0011 120.7336) (width 0.2032) (layer "F.Cu") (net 10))
 (segment (start 144.7511 117.2036) (end 144.7511 119.0036) (width 0.2) (layer "F.Cu") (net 10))
 (segment (start 148.7111 119.0036) (end 144.7511 119.0036) (width 0.2032) (layer "F.Cu") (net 10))
 (segment (start 156.0011 91.9536) (end 151.3011 91.9536) (width 0.2032) (layer "F.Cu") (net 8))
 (segment (start 153.2011 98.0536) (end 156.0011 98.0536) (width 0.2032) (layer "F.Cu") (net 3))
 (segment (start 151.3011 99.9536) (end 153.2011 98.0536) (width 0.2032) (layer "F.Cu") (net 3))
 (segment (start 151.3011 119.9536) (end 153.2011 118.0536) (width 0.2032) (layer "F.Cu") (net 12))
 (segment (start 153.2011 118.0536) (end 156.0011 118.0536) (width 0.2032) (layer "F.Cu") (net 12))
 (segment (start 156.0011 90.0536) (end 154.2711 88.3236) (width 0.2032) (layer "F.Cu") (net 11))
 (segment (start 154.2711 88.3236) (end 154.2711 85.0036) (width 0.2032) (layer "F.Cu") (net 11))
 (segment (start 153.4911 102.4636) (end 156.0011 99.9536) (width 0.2032) (layer "F.Cu") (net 9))
 (segment (start 153.0011 102.4636) (end 153.4911 102.4636) (width 0.2) (layer "F.Cu") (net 9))
 (segment (start 156.0011 123.2736) (end 154.2711 125.0036) (width 0.2032) (layer "F.Cu") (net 13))
 (segment (start 156.0011 119.9536) (end 156.0011 123.2736) (width 0.2032) (layer "F.Cu") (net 13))
 (segment (start 151.3011 111.9536) (end 156.0011 111.9536) (width 0.2032) (layer "F.Cu") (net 5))
 (segment (start 153.4911 107.5436) (end 153.0011 107.5436) (width 0.2) (layer "F.Cu") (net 6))
 (segment (start 156.0011 110.0536) (end 153.4911 107.5436) (width 0.2) (layer "F.Cu") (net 6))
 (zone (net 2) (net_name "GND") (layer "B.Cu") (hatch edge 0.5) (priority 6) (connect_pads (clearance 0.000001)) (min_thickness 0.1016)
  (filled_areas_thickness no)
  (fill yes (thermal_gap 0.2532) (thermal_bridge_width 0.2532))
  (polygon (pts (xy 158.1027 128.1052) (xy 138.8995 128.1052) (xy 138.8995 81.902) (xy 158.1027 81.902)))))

